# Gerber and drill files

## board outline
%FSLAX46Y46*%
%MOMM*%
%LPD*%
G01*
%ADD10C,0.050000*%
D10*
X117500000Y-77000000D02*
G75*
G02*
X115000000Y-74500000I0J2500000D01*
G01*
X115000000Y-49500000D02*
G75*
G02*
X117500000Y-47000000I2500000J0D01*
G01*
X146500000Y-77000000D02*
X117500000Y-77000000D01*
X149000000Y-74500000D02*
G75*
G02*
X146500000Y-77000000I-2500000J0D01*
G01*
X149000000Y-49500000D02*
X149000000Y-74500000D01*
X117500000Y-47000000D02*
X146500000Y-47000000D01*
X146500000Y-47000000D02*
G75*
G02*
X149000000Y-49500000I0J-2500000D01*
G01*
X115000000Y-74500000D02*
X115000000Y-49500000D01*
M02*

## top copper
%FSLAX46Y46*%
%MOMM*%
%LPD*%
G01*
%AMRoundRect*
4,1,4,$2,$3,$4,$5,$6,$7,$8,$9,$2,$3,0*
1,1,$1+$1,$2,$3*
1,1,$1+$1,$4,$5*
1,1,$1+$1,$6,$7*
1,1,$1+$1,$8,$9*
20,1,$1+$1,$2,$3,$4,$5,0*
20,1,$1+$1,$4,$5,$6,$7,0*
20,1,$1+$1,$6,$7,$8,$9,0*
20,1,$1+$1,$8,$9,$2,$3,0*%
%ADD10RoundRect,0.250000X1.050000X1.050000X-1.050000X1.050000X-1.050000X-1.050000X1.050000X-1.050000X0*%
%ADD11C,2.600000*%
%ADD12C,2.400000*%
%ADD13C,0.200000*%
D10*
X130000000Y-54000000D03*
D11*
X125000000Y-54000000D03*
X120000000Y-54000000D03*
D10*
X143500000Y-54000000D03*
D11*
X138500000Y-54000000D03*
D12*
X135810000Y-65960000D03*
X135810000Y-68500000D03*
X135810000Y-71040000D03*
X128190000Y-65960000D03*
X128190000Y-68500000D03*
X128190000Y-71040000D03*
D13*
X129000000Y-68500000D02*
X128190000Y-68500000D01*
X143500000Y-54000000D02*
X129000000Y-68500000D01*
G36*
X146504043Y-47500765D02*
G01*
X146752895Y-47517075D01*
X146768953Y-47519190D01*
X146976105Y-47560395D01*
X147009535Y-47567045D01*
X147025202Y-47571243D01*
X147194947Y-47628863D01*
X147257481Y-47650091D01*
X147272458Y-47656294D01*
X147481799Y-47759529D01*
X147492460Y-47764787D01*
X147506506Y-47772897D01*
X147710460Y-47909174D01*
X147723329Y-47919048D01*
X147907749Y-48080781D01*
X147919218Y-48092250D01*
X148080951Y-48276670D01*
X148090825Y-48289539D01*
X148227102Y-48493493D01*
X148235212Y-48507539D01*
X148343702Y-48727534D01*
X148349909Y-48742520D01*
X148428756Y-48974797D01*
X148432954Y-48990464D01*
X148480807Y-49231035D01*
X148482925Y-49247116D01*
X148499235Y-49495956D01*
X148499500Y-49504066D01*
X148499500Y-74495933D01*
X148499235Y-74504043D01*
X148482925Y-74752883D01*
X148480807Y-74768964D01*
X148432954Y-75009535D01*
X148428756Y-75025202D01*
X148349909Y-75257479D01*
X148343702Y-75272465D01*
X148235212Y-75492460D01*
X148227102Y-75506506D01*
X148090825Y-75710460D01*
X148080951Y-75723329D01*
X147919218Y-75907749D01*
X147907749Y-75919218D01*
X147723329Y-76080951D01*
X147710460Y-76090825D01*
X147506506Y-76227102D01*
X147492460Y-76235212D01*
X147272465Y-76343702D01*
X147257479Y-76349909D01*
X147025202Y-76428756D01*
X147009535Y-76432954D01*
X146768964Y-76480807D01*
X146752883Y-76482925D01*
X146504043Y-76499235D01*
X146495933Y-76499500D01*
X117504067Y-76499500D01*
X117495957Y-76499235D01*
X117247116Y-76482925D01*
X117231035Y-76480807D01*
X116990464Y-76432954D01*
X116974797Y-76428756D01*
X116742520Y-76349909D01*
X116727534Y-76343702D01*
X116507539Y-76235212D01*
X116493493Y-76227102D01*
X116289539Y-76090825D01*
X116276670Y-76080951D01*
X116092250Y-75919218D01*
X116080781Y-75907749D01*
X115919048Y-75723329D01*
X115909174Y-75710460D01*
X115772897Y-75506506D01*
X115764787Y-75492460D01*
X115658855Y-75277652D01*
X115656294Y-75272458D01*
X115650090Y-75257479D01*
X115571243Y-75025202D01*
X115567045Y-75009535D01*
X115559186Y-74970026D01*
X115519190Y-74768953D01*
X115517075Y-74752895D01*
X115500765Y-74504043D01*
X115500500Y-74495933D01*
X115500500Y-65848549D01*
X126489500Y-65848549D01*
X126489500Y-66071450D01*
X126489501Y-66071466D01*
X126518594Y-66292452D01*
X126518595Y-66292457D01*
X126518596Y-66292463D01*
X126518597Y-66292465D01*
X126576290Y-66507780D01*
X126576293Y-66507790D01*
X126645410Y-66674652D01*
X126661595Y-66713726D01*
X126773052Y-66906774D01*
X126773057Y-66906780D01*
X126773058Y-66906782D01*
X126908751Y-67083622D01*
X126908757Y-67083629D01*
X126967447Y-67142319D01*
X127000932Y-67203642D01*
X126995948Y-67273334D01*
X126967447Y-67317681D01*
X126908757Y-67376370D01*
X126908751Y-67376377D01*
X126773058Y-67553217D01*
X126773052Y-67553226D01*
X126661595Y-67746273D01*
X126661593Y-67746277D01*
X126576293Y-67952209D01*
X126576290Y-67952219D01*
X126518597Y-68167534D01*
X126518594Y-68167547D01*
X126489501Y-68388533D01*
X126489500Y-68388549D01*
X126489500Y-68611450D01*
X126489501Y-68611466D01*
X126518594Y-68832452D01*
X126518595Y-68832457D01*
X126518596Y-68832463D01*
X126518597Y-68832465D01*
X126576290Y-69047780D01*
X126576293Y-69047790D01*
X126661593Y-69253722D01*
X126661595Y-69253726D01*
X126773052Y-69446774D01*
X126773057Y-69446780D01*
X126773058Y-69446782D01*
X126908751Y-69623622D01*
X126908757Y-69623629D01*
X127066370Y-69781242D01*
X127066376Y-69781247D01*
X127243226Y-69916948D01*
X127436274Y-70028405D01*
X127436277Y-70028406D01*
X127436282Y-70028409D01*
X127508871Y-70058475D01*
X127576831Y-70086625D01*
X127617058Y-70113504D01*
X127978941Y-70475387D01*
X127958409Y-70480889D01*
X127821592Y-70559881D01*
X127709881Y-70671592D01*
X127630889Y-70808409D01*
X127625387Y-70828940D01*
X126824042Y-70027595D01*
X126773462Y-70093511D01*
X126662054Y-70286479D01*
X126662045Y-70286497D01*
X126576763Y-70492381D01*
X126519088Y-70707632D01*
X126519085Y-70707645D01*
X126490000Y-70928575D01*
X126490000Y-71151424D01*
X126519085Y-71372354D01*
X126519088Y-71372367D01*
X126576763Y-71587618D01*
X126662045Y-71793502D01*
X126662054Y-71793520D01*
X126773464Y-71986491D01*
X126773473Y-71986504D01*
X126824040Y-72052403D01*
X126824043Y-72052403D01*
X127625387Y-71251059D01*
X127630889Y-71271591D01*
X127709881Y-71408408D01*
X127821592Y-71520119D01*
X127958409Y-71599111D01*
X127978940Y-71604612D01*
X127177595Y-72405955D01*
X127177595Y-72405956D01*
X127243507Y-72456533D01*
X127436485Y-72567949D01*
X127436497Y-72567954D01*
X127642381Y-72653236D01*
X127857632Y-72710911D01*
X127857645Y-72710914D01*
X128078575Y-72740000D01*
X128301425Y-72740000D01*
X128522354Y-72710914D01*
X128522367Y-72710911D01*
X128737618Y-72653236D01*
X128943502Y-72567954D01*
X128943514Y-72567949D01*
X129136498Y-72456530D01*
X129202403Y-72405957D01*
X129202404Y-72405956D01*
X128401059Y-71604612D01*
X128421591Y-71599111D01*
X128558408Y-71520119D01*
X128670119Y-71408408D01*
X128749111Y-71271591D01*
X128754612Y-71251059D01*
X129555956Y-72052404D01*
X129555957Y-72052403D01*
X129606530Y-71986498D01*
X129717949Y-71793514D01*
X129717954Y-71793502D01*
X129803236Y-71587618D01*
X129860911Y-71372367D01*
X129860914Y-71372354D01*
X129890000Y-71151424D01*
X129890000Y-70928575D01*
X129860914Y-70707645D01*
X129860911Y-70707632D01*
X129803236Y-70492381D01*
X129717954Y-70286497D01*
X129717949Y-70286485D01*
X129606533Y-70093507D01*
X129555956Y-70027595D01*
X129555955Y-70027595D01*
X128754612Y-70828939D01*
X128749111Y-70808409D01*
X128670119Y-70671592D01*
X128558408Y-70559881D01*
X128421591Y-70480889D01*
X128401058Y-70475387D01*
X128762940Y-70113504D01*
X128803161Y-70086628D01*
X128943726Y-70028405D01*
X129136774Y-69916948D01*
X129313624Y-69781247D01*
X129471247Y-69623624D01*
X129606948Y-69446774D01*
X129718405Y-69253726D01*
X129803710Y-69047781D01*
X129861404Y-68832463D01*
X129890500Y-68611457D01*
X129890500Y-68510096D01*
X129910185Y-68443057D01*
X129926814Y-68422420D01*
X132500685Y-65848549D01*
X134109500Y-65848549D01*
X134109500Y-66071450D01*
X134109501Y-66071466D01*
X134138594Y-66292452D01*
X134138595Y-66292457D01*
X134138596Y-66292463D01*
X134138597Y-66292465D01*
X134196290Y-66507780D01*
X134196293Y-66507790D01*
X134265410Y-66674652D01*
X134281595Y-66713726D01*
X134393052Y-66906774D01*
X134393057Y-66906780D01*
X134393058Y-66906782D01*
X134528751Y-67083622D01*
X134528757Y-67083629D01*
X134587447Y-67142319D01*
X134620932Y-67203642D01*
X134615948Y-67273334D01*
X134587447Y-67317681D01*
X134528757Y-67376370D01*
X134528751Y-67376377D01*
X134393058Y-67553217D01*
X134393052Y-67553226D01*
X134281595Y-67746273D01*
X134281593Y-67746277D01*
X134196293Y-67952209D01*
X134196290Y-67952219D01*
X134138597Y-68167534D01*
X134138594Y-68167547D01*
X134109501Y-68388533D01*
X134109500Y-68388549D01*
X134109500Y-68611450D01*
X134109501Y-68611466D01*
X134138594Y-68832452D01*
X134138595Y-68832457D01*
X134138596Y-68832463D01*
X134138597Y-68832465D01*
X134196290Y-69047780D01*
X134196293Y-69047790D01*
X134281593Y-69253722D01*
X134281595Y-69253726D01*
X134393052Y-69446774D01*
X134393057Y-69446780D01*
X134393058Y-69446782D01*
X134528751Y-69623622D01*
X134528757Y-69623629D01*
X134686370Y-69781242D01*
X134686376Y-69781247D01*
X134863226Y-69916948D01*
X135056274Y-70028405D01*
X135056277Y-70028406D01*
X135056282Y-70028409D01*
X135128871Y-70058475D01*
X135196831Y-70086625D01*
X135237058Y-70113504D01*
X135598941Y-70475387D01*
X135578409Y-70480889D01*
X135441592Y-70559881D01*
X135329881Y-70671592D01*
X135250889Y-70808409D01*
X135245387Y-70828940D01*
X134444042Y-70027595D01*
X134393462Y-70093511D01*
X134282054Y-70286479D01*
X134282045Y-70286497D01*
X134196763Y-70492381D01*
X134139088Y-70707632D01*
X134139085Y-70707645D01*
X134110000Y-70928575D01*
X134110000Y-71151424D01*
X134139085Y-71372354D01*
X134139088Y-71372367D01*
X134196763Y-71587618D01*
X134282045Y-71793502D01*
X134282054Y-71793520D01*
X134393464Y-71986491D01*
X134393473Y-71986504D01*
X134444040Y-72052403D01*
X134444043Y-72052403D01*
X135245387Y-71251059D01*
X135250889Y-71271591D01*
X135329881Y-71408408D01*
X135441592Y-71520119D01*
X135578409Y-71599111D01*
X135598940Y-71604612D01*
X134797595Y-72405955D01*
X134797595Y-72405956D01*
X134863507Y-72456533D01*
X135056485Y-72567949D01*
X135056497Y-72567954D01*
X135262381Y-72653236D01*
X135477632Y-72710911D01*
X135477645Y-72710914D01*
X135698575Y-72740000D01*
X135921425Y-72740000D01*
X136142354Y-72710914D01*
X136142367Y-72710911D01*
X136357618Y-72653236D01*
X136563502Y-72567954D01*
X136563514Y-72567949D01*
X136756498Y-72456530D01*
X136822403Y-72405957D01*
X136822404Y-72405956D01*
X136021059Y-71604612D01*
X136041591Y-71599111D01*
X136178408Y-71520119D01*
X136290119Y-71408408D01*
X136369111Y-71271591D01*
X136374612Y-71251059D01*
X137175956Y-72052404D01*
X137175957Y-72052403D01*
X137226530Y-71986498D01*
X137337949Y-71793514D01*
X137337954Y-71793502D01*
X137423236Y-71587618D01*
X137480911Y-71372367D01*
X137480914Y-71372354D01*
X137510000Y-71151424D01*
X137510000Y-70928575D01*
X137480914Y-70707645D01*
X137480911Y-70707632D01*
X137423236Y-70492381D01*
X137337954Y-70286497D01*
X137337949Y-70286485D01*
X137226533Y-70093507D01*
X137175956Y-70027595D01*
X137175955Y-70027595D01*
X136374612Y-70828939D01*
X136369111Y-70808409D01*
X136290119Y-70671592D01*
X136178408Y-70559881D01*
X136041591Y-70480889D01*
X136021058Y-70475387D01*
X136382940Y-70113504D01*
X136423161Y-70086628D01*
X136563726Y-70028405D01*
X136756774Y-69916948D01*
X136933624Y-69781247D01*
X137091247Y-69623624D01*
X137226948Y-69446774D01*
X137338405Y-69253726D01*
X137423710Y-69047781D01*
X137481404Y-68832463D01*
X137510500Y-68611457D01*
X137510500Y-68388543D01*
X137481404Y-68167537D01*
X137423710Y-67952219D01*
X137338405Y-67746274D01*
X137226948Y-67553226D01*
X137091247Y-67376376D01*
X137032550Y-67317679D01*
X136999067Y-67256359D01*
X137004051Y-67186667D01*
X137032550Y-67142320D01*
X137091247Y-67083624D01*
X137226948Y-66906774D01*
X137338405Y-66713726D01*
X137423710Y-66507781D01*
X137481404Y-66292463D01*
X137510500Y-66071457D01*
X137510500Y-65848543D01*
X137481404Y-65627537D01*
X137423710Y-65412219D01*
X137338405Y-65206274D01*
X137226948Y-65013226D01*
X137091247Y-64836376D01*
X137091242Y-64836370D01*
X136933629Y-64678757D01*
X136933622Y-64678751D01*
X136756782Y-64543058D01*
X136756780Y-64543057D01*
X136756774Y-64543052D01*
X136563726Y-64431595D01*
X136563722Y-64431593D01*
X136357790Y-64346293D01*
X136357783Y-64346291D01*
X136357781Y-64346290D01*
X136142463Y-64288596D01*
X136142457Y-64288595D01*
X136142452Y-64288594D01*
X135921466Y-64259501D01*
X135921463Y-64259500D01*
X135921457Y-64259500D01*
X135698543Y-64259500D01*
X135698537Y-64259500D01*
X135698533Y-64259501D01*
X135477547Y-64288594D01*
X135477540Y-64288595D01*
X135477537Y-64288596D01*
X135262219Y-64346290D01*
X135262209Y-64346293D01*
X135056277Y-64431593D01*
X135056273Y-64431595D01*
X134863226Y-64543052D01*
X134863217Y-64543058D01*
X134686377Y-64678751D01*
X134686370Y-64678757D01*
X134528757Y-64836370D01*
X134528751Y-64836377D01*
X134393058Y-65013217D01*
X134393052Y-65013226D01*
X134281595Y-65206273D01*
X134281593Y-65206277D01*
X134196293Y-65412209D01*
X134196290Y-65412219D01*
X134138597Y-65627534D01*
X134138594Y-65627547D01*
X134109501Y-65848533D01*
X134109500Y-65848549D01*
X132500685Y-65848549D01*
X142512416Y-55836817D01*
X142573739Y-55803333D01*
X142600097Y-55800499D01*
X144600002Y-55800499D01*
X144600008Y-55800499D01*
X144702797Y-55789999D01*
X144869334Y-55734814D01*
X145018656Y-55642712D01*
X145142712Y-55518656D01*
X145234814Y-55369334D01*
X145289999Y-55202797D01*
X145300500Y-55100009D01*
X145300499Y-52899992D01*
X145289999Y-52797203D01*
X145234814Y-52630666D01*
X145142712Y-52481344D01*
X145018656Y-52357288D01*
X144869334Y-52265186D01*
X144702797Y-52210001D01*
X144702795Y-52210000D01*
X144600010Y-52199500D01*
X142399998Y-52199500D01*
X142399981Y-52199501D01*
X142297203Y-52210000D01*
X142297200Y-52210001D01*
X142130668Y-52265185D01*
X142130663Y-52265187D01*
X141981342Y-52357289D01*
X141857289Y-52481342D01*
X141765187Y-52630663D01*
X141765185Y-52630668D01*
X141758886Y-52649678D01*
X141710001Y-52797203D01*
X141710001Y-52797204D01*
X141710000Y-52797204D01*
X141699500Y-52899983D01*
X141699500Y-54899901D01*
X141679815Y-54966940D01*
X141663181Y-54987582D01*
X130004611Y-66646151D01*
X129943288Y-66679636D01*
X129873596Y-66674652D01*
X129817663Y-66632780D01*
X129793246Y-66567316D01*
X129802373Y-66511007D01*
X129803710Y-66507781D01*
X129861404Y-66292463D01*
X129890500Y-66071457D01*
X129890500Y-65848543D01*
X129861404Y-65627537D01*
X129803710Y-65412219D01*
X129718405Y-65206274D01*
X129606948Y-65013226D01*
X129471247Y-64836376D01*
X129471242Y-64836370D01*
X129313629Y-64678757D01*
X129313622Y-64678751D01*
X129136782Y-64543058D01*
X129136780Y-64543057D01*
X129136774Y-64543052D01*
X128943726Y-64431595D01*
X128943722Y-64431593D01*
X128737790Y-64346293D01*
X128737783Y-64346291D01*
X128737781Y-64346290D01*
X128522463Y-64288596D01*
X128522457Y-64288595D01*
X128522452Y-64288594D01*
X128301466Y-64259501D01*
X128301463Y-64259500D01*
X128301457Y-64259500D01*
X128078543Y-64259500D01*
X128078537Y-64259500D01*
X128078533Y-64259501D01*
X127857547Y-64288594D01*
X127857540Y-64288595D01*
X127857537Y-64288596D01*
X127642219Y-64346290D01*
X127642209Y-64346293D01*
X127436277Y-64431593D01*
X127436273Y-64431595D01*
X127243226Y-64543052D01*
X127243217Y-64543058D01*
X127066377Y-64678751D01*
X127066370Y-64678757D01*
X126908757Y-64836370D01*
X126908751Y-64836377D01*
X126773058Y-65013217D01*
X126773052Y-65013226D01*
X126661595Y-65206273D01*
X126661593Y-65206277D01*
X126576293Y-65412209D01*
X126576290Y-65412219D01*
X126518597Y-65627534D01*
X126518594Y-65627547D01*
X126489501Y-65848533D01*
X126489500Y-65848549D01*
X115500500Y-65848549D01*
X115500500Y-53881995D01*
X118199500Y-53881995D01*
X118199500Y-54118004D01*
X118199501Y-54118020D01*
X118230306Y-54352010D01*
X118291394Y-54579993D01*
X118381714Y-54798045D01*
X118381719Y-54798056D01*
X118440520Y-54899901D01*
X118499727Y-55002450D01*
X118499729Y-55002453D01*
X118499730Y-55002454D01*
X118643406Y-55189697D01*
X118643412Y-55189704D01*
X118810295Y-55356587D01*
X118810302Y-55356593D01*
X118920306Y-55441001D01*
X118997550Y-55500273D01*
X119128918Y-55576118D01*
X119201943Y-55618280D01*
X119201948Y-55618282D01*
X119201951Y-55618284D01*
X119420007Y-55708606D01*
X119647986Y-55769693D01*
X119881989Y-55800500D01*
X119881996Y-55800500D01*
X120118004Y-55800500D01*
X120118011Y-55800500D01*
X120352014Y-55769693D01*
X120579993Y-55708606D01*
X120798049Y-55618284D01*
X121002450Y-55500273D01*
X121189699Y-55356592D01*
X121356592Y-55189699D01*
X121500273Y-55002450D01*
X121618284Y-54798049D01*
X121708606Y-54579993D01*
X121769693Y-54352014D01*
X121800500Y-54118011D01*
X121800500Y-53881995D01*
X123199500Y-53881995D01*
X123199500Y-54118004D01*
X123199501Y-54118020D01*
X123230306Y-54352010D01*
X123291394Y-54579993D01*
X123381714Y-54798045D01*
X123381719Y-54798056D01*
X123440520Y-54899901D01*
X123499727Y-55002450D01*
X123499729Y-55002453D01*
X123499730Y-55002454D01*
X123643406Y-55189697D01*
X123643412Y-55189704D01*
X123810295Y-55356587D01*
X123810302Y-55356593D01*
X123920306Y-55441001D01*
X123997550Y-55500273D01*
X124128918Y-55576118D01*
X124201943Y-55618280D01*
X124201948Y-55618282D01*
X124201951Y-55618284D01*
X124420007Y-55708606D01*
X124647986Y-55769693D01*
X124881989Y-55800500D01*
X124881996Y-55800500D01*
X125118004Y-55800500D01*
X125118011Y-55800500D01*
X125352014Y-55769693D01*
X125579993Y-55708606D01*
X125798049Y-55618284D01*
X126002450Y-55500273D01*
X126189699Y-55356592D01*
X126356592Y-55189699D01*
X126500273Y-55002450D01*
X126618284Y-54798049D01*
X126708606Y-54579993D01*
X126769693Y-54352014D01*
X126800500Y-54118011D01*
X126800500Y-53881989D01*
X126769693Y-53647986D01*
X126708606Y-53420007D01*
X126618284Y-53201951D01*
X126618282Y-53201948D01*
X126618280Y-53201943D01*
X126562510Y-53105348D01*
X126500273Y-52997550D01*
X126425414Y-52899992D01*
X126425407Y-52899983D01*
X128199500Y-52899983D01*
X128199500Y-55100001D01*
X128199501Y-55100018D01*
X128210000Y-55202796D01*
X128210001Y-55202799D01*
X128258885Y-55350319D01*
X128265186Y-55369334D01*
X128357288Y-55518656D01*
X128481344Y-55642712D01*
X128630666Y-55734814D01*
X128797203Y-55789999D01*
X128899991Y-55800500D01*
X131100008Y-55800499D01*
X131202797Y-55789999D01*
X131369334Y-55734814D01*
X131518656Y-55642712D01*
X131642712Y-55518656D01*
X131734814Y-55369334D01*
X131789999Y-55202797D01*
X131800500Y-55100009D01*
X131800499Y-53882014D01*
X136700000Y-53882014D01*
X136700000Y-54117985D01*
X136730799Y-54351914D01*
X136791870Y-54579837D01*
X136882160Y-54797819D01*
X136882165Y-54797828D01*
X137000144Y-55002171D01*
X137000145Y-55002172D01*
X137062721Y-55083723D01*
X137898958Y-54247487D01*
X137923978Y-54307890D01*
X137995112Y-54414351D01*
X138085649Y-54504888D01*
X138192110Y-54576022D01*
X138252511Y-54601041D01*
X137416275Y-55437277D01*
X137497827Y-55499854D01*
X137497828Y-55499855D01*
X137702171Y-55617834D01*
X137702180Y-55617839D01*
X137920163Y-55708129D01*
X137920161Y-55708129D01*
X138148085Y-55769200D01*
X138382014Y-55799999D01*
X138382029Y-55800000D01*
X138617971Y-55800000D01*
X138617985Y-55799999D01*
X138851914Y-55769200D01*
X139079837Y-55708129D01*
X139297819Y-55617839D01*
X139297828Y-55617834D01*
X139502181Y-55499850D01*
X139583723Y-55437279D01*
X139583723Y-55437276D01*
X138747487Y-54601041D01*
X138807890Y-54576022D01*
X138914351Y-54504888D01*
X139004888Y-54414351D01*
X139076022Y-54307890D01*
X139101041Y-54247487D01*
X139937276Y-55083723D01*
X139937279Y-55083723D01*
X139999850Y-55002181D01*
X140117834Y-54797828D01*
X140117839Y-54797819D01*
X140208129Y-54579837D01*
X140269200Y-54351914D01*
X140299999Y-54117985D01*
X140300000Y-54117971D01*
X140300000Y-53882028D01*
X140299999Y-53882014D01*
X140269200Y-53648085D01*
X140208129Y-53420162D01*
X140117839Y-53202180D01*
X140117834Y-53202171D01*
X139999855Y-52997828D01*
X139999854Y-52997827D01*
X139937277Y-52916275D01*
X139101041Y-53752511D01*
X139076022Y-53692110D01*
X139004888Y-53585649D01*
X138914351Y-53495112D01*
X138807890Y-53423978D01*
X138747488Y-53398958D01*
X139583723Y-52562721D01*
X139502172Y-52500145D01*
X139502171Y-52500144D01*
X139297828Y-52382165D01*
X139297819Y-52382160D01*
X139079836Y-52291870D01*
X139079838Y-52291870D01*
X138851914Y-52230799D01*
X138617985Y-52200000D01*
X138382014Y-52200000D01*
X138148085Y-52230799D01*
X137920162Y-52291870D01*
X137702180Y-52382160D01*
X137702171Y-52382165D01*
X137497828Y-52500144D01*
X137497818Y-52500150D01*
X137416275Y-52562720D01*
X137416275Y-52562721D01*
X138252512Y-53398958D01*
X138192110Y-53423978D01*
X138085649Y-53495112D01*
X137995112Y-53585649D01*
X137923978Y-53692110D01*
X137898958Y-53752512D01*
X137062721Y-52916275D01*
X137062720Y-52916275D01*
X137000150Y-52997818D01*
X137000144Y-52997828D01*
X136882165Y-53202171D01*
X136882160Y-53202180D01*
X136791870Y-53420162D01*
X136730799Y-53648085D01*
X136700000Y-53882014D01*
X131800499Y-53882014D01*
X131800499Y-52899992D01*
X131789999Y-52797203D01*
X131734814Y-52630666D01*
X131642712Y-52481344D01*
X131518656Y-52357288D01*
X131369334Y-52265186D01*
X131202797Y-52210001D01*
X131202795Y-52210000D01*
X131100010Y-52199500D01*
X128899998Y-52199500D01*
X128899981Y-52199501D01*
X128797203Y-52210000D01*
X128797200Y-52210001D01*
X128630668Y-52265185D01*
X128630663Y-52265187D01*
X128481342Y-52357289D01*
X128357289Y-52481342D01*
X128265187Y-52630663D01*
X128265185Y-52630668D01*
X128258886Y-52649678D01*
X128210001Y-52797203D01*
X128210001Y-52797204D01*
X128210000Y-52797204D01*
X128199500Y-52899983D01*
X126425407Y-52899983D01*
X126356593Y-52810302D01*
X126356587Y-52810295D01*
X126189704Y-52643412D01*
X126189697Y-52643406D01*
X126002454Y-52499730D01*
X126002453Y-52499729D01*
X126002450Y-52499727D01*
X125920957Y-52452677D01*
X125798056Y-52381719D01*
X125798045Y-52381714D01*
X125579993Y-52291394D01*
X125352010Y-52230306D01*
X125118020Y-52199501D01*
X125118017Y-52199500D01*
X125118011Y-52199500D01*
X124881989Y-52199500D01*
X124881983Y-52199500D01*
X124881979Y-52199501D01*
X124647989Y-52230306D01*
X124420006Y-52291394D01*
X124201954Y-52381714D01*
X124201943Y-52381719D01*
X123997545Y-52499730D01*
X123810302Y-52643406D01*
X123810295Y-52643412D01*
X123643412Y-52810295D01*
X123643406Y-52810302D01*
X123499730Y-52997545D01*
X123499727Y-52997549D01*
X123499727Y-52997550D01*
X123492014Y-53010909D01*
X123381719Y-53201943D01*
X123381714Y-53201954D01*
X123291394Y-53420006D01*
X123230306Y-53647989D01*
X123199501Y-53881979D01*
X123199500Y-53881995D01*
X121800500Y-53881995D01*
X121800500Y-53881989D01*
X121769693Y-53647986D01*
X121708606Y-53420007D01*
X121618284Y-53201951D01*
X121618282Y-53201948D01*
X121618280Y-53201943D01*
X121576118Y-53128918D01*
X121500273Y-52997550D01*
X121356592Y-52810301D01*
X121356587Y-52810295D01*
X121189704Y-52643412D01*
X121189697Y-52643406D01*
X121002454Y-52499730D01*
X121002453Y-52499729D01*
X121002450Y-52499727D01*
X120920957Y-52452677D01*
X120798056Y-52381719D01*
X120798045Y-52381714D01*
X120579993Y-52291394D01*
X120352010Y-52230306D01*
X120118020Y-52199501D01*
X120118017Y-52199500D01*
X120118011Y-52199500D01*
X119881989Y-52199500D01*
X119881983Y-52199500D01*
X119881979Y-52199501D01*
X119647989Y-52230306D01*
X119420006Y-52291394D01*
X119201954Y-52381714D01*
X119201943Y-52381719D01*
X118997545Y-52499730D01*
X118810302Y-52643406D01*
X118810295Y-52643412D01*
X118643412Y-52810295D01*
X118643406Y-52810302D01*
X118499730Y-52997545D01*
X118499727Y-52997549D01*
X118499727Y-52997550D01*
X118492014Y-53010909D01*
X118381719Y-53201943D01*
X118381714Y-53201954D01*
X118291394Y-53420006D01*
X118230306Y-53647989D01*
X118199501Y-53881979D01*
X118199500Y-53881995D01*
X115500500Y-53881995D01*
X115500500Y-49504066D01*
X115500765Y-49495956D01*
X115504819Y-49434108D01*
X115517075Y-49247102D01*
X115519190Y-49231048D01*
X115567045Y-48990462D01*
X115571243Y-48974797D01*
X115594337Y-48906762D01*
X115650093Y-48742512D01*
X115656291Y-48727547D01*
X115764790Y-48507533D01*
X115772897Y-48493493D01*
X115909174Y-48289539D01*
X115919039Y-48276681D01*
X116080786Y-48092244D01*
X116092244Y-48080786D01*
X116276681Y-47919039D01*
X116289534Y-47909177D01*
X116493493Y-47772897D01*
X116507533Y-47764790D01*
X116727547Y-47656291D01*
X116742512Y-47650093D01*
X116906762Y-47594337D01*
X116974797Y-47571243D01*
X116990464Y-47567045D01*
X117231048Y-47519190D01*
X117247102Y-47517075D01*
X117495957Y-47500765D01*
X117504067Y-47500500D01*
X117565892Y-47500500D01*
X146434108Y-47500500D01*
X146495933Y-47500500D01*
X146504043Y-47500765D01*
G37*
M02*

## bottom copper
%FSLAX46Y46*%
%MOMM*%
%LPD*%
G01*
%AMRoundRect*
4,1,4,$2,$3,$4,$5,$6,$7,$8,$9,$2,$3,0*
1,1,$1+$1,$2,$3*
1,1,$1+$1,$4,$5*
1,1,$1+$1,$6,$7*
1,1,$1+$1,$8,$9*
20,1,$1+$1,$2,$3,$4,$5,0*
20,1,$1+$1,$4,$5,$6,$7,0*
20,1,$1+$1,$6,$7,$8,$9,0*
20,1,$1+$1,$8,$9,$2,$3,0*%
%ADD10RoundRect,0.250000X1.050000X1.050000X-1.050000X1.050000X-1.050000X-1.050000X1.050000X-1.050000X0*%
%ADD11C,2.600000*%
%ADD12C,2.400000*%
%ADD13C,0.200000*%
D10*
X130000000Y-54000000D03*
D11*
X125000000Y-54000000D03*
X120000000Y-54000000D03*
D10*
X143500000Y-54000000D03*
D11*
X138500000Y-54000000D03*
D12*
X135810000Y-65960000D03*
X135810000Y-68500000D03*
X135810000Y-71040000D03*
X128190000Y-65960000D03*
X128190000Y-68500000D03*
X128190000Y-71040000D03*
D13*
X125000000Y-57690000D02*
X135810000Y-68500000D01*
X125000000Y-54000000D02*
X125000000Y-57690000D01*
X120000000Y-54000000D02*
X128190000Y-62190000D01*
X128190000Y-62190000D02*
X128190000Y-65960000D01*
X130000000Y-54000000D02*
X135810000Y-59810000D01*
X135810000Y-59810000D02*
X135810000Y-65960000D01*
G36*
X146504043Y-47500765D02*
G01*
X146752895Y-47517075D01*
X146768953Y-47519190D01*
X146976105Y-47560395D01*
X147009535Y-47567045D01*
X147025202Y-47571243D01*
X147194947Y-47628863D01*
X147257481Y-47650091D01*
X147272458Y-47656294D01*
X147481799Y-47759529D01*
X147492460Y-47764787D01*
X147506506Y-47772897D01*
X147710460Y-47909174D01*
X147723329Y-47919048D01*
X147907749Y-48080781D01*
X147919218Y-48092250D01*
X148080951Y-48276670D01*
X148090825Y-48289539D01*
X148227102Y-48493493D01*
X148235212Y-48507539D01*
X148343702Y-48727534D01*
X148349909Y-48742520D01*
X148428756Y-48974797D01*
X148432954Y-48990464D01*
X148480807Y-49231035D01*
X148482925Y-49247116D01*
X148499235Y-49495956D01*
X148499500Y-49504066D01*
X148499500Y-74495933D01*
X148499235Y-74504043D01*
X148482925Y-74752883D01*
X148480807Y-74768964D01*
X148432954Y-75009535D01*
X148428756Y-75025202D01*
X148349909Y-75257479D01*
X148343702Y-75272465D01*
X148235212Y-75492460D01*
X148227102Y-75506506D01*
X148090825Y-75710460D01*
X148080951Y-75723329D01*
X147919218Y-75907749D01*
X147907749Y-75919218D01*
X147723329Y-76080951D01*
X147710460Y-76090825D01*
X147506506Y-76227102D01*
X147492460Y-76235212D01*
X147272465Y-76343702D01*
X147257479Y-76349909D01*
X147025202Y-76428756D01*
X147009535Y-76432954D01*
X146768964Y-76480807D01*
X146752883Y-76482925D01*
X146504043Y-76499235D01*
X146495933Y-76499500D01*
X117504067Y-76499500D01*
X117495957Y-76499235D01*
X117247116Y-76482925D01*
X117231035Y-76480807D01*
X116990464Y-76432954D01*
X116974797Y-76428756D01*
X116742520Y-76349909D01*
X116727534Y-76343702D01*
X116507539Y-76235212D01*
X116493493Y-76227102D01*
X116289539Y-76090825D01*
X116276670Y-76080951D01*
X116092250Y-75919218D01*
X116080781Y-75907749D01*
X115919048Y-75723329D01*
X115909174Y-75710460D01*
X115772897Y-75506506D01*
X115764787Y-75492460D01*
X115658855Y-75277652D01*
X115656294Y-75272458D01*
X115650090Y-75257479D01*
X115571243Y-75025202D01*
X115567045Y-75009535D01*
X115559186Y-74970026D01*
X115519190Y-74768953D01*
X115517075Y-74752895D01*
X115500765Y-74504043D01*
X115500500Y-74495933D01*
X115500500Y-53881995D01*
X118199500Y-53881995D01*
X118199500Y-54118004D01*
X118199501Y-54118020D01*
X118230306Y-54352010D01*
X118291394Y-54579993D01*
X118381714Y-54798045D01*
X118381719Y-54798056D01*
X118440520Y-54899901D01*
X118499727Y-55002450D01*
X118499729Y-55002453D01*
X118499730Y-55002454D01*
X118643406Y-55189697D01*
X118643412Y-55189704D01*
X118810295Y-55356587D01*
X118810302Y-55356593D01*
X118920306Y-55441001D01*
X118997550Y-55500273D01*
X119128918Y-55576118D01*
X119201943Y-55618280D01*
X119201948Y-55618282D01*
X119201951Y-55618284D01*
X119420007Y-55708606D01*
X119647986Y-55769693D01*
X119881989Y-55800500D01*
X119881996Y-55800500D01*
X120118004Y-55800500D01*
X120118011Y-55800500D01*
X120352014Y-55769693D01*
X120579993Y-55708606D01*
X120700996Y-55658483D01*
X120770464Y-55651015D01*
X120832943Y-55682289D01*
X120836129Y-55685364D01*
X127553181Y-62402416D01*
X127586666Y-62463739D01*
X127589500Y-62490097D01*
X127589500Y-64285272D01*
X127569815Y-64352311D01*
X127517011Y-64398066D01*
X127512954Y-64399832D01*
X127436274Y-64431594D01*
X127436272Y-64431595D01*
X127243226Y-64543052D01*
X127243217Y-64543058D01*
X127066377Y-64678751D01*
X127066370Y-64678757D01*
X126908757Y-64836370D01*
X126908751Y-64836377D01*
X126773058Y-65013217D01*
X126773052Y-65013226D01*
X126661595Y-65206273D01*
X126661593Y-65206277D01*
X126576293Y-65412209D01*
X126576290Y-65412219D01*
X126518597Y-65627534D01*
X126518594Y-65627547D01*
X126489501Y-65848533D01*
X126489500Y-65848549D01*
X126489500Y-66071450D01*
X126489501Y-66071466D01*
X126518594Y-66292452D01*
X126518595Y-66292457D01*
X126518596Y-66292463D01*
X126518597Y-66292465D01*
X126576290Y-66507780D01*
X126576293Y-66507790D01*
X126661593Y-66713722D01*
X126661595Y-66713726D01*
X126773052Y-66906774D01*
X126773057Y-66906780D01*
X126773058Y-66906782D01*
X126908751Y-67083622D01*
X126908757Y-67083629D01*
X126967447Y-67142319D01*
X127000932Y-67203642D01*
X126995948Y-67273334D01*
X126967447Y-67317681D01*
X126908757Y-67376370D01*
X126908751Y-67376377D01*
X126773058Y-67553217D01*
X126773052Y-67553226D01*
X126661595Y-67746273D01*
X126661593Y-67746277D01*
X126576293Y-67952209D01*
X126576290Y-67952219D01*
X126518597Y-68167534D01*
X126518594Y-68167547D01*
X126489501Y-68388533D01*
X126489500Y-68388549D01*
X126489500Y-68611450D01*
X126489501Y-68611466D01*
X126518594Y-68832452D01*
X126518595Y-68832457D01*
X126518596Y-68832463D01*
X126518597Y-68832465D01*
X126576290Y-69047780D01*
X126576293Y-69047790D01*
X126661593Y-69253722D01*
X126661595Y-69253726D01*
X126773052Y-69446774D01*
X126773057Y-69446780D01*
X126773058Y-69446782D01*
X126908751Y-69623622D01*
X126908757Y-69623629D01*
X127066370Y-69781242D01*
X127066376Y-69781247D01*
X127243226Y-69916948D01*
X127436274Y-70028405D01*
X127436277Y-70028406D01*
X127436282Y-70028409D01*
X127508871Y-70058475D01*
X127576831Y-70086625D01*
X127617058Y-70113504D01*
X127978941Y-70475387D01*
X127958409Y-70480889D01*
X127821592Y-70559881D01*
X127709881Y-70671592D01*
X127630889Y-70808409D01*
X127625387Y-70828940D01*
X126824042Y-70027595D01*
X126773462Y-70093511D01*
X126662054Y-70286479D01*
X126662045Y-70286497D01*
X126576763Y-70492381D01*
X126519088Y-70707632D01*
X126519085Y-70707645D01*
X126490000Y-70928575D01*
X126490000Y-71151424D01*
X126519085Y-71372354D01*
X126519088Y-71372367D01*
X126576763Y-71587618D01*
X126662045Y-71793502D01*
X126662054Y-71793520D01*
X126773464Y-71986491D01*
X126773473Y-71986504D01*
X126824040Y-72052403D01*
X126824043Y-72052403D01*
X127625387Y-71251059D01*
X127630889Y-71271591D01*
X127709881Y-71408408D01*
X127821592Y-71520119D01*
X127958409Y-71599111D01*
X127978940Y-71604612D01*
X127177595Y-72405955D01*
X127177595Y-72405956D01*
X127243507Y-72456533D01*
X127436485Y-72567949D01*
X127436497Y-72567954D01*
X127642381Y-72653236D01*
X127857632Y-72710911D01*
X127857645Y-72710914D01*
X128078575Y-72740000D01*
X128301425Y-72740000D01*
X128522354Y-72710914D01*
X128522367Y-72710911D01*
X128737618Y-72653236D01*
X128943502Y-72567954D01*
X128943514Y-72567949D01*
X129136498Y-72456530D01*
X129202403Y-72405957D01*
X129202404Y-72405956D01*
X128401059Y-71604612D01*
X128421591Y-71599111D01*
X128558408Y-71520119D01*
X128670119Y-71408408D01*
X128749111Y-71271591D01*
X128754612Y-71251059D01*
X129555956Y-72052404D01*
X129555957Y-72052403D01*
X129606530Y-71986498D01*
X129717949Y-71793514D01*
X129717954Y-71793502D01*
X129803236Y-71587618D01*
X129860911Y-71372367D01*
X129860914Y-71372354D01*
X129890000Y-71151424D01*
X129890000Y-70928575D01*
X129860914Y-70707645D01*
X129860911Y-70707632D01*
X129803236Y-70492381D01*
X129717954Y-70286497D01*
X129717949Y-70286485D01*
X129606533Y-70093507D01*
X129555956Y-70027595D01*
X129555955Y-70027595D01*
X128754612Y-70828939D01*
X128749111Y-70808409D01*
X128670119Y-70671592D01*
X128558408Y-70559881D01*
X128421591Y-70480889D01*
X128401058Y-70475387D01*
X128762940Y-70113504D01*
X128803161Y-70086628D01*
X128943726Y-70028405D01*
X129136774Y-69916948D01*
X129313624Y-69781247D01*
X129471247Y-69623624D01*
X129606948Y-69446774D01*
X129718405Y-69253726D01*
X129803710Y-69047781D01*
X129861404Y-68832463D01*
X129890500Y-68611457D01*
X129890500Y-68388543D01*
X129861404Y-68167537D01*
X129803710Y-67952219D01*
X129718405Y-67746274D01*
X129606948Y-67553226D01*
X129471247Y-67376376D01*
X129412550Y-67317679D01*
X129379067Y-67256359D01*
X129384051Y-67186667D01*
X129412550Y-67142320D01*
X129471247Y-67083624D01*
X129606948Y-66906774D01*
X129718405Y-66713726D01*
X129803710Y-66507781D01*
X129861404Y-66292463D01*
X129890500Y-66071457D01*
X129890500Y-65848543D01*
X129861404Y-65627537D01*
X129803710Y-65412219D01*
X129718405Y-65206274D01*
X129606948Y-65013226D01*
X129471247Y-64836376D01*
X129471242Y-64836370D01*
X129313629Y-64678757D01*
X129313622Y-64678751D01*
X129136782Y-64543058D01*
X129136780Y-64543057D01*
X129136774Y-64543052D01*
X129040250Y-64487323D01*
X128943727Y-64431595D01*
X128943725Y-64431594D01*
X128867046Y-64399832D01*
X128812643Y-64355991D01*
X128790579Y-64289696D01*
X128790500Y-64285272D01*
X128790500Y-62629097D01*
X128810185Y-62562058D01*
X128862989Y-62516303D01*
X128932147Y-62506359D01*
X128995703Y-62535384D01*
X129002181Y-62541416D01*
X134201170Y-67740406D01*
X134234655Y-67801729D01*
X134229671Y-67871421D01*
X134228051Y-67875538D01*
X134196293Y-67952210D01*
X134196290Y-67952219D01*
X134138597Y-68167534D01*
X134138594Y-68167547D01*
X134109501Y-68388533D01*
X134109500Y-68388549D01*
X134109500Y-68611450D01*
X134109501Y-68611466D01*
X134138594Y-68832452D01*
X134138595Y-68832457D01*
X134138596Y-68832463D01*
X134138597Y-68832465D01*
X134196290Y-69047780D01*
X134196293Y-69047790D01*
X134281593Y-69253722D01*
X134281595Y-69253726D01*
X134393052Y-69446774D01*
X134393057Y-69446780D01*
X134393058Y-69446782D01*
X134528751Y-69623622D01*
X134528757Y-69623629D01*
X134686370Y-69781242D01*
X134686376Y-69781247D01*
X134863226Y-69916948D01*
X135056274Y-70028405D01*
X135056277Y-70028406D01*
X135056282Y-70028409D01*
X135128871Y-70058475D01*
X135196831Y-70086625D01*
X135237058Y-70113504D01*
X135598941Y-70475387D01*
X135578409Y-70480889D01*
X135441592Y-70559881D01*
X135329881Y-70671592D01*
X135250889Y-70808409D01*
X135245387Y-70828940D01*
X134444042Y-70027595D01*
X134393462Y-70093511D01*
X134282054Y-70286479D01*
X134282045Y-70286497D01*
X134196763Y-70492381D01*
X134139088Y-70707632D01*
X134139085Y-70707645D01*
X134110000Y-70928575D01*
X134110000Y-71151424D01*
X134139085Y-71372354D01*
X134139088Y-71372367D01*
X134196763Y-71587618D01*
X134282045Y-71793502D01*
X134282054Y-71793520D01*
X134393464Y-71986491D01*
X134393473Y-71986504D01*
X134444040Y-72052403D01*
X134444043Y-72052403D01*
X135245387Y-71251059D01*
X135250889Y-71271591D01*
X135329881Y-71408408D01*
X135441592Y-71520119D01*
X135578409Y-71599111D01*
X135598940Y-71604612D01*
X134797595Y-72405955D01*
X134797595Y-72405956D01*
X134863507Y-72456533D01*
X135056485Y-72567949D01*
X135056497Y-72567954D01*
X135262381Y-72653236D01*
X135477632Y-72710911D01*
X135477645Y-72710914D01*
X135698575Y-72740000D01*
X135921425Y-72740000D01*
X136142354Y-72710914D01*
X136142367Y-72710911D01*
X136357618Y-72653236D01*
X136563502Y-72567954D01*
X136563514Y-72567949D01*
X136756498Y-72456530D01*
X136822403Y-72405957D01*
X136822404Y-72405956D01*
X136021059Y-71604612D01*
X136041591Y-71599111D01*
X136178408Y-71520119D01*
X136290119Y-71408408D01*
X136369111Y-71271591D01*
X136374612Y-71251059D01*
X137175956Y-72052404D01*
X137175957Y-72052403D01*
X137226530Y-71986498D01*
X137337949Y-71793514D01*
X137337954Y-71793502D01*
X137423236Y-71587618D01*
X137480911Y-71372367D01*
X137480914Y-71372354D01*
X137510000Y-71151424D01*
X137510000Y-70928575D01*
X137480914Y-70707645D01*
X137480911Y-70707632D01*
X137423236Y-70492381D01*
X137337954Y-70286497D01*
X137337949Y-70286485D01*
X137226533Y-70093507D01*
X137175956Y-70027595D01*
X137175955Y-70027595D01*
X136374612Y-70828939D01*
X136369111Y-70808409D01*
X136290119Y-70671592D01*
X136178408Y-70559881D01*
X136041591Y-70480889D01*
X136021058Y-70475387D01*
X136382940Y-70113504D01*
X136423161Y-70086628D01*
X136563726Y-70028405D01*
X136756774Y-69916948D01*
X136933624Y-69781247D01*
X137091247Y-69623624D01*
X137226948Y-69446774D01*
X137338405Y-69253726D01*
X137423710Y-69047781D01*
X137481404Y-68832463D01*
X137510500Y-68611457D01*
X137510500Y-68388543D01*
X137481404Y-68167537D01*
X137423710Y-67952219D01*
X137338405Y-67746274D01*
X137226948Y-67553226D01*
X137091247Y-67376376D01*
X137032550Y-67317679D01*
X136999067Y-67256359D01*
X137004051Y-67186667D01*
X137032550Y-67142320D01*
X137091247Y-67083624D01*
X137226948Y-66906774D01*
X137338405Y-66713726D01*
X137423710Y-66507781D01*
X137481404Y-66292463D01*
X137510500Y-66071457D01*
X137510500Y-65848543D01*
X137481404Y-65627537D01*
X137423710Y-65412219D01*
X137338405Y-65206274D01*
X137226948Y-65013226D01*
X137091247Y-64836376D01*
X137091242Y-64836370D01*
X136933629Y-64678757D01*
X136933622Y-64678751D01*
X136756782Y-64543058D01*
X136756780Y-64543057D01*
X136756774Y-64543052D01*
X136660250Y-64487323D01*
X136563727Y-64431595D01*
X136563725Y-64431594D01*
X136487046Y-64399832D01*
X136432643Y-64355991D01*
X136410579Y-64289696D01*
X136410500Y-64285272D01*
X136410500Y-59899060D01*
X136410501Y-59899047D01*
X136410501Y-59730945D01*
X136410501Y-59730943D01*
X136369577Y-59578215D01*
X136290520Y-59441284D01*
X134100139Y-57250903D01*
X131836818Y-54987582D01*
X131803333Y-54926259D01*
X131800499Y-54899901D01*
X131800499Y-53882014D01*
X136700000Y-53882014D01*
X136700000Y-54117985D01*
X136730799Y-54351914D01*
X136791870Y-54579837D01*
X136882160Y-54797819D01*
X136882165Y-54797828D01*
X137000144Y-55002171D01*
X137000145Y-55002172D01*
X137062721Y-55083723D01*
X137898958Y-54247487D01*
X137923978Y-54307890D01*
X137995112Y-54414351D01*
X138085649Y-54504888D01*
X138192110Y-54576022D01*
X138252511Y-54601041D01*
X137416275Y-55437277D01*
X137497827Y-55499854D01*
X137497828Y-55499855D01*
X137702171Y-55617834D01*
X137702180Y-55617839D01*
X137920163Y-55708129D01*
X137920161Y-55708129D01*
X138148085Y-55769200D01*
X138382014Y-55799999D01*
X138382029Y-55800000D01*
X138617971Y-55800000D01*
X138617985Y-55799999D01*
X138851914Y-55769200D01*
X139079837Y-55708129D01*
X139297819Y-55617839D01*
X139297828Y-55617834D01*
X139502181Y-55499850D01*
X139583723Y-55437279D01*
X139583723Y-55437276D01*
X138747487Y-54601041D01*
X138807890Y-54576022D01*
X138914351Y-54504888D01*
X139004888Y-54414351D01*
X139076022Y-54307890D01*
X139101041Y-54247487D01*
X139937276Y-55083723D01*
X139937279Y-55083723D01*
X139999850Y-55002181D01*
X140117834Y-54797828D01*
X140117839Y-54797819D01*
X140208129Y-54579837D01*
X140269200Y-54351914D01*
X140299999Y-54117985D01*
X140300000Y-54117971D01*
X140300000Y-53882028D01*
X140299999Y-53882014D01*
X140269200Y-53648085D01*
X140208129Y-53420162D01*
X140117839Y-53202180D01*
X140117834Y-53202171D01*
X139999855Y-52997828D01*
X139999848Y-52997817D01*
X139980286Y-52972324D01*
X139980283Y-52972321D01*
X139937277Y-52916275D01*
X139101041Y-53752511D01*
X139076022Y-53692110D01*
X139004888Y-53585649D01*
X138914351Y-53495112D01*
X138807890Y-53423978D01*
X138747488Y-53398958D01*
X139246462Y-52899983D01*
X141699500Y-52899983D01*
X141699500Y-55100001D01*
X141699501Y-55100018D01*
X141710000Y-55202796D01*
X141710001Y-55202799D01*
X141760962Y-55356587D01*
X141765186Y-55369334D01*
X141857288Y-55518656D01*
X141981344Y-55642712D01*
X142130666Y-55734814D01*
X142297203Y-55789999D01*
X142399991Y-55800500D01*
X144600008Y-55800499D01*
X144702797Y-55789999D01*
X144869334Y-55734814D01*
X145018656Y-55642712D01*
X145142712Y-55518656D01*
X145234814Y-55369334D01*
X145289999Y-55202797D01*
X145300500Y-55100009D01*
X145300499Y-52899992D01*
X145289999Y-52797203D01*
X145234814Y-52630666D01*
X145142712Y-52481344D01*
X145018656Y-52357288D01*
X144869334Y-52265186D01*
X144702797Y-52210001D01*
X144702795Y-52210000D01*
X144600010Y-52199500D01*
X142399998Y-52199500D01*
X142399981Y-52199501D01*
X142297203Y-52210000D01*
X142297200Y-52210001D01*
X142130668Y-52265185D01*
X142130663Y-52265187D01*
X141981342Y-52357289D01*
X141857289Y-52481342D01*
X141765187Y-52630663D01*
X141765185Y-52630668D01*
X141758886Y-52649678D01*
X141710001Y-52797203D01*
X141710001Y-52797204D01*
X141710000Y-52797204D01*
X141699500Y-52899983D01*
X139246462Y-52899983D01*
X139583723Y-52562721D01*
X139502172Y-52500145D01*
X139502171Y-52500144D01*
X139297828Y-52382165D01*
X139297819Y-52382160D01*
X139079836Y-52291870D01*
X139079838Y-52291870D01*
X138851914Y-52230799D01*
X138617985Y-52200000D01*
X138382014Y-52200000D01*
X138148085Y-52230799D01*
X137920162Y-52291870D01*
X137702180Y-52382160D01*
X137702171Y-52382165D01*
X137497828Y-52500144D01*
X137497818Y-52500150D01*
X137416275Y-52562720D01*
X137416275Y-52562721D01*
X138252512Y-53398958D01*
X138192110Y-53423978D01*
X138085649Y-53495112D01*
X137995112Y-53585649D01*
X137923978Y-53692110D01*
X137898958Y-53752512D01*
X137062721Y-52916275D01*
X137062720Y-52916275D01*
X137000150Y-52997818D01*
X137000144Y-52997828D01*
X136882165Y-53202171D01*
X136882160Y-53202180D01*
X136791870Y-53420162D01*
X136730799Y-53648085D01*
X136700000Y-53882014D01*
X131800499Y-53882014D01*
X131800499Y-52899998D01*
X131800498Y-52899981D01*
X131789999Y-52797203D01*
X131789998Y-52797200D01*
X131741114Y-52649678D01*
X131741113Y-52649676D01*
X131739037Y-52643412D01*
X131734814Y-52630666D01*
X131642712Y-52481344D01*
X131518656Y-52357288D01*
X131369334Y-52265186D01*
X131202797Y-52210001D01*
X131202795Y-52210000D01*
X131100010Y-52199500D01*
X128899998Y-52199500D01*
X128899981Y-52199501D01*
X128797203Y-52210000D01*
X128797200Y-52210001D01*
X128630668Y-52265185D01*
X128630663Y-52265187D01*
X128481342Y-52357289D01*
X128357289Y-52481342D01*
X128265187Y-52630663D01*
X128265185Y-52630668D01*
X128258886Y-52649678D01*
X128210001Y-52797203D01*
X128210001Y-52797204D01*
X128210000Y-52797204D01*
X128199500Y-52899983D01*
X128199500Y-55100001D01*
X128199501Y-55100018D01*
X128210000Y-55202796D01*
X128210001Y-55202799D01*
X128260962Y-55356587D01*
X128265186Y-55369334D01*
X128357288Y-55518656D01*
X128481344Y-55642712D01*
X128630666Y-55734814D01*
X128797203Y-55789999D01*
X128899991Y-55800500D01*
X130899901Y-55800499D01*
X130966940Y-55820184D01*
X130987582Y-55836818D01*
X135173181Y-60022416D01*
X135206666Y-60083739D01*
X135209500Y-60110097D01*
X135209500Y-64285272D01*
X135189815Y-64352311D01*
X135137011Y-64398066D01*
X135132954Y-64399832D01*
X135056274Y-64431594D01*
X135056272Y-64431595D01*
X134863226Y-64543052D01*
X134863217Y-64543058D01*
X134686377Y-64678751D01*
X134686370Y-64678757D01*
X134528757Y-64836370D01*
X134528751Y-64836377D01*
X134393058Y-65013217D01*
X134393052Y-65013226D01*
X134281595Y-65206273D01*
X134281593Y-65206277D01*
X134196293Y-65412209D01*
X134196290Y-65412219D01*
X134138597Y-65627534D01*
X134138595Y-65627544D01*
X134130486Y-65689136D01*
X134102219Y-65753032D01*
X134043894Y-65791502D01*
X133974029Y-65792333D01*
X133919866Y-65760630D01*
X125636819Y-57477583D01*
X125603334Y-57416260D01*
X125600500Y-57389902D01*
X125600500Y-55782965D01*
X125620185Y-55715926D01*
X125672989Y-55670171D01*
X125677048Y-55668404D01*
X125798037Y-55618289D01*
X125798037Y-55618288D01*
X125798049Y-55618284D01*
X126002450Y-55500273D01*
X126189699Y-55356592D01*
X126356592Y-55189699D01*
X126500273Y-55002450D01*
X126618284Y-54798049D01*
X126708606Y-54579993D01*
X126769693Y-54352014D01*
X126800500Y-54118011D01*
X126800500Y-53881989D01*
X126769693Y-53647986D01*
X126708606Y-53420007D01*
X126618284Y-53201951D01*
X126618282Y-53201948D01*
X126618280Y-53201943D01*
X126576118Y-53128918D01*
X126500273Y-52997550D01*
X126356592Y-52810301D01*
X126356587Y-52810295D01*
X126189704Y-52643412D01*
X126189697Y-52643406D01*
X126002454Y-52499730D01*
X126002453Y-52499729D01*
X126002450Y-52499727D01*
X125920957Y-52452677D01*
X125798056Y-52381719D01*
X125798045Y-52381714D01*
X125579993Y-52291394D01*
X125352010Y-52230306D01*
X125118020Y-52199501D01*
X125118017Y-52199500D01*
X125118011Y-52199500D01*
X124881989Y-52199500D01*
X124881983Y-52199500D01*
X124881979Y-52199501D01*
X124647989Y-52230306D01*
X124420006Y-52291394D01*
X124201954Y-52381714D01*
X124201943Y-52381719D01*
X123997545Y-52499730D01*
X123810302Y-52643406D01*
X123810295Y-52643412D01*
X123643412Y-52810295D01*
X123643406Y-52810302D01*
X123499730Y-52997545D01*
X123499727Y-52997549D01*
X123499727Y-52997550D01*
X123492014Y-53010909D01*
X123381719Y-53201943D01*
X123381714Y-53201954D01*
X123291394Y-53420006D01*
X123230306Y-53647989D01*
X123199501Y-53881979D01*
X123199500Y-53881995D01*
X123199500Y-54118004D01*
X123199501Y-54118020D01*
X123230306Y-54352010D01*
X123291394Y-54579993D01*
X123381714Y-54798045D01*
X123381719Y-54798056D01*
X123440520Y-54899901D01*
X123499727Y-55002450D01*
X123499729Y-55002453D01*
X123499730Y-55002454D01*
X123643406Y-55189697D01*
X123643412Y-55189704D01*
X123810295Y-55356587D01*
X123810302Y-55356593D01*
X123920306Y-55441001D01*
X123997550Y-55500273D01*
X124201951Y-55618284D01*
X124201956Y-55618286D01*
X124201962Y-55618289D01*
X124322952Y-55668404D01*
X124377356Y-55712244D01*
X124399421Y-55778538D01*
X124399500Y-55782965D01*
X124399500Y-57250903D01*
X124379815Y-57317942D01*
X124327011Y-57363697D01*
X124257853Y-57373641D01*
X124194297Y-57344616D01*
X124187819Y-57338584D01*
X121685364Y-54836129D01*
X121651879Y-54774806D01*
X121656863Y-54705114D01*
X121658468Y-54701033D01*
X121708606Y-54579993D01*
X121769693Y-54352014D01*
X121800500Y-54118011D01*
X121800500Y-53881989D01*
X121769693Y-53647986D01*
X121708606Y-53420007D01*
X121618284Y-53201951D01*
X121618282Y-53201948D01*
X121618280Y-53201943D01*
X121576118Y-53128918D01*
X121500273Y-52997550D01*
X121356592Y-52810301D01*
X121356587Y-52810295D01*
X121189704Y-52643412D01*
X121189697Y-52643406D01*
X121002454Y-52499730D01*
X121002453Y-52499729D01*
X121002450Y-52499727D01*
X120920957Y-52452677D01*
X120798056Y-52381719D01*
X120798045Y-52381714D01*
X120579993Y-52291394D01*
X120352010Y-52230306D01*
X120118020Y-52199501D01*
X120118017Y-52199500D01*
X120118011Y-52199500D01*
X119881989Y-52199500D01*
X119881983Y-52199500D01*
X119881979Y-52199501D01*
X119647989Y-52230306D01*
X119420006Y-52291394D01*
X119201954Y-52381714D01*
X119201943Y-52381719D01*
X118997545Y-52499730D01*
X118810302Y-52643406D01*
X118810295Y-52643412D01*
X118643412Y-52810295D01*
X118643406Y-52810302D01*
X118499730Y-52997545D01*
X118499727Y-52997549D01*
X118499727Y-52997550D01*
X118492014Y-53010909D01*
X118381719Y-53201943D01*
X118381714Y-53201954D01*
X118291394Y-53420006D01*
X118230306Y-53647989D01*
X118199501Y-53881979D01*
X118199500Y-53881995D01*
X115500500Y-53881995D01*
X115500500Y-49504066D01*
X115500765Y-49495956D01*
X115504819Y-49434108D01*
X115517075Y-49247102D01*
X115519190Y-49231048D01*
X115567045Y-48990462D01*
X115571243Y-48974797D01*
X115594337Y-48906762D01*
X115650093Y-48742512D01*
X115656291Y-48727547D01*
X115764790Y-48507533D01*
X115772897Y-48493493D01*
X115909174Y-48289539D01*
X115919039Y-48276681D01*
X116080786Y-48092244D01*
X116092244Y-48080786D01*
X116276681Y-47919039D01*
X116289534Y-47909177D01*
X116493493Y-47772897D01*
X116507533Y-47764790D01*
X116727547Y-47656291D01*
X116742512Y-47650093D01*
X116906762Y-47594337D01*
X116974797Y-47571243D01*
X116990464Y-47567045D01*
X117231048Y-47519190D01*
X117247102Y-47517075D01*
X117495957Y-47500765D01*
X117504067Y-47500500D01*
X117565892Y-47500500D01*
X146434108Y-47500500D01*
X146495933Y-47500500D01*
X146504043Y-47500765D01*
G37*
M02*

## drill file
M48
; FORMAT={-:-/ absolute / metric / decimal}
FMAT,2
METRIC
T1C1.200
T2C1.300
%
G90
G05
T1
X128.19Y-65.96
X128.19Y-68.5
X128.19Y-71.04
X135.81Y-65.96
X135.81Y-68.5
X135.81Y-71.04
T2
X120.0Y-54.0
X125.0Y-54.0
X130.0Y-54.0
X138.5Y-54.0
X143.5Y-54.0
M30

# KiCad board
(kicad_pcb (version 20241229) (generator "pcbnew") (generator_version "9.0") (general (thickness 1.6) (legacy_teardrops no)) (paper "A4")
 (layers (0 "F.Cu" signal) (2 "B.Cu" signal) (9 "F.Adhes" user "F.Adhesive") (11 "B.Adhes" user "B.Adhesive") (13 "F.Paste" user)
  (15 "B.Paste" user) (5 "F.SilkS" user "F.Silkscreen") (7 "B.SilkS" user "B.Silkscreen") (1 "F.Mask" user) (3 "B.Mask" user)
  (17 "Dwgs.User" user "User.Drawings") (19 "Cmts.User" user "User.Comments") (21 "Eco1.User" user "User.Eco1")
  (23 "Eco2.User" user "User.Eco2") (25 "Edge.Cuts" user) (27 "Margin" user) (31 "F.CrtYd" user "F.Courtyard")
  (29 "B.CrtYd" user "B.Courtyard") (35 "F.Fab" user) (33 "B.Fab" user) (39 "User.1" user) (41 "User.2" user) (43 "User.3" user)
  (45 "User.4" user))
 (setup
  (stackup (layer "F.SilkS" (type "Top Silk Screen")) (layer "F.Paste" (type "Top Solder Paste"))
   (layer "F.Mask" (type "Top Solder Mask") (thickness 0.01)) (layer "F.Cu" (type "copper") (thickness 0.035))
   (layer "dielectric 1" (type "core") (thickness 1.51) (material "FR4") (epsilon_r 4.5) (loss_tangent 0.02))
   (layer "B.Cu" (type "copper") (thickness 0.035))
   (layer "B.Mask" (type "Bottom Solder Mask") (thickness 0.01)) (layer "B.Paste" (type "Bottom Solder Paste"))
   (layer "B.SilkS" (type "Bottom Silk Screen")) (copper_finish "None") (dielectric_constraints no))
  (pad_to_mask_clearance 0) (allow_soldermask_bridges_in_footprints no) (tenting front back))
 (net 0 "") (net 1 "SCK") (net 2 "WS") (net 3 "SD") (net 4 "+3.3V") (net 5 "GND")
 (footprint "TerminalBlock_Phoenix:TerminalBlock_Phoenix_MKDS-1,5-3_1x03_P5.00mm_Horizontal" (layer "F.Cu") (at 130 54 180)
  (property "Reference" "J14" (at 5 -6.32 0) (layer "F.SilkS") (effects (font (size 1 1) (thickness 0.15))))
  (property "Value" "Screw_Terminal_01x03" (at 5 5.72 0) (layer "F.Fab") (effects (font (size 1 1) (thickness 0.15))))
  (pad "1" thru_hole roundrect (at 0 0 180) (size 2.6 2.6) (drill 1.3) (layers "*.Cu" "*.Mask") (remove_unused_layers no)
   (roundrect_rratio 0.096154) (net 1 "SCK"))
  (pad "2" thru_hole circle (at 5 0 180) (size 2.6 2.6) (drill 1.3) (layers "*.Cu" "*.Mask") (remove_unused_layers no) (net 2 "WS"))
  (pad "3" thru_hole circle (at 10 0 180) (size 2.6 2.6) (drill 1.3) (layers "*.Cu" "*.Mask") (remove_unused_layers no) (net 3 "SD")))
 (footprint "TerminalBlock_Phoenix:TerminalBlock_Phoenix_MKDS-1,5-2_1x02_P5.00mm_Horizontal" (layer "F.Cu") (at 143.5 54 180)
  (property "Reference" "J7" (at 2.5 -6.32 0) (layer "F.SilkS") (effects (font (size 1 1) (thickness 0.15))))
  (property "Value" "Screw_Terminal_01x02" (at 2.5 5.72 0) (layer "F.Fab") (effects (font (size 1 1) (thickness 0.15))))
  (pad "1" thru_hole roundrect (at 0 0 180) (size 2.6 2.6) (drill 1.3) (layers "*.Cu" "*.Mask") (remove_unused_layers no)
   (roundrect_rratio 0.096154) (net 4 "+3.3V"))
  (pad "2" thru_hole circle (at 5 0 180) (size 2.6 2.6) (drill 1.3) (layers "*.Cu" "*.Mask") (remove_unused_layers no) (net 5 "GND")))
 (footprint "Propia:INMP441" (layer "F.Cu") (at 132 68.5)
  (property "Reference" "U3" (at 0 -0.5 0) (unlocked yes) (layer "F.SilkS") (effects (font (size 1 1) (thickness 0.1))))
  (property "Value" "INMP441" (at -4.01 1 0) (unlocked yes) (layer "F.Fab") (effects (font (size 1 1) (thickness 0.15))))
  (pad "1" thru_hole circle (at 3.81 -2.54) (size 2.4 2.4) (drill 1.2) (layers "*.Cu" "*.Mask") (remove_unused_layers no) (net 1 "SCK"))
  (pad "2" thru_hole circle (at 3.81 0) (size 2.4 2.4) (drill 1.2) (layers "*.Cu" "*.Mask") (remove_unused_layers no) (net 2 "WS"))
  (pad "3" thru_hole circle (at 3.81 2.54) (size 2.4 2.4) (drill 1.2) (layers "*.Cu" "*.Mask") (remove_unused_layers no) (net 5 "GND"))
  (pad "4" thru_hole circle (at -3.81 -2.54) (size 2.4 2.4) (drill 1.2) (layers "*.Cu" "*.Mask") (remove_unused_layers no) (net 3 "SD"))
  (pad "5" thru_hole circle (at -3.81 0) (size 2.4 2.4) (drill 1.2) (layers "*.Cu" "*.Mask") (remove_unused_layers no) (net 4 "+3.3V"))
  (pad "6" thru_hole circle (at -3.81 2.54) (size 2.4 2.4) (drill 1.2) (layers "*.Cu" "*.Mask") (remove_unused_layers no) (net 5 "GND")))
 (gr_arc (start 117.5 77) (mid 115.732233 76.267767) (end 115 74.5) (stroke (width 0.05) (type default)) (layer "Edge.Cuts"))
 (gr_arc (start 115 49.5) (mid 115.732233 47.732233) (end 117.5 47) (stroke (width 0.05) (type default)) (layer "Edge.Cuts"))
 (gr_line (start 146.5 77) (end 117.5 77) (stroke (width 0.05) (type default)) (layer "Edge.Cuts"))
 (gr_arc (start 149 74.5) (mid 148.267767 76.267767) (end 146.5 77) (stroke (width 0.05) (type default)) (layer "Edge.Cuts"))
 (gr_line (start 149 49.5) (end 149 74.5) (stroke (width 0.05) (type default)) (layer "Edge.Cuts"))
 (gr_line (start 117.5 47) (end 146.5 47) (stroke (width 0.05) (type default)) (layer "Edge.Cuts"))
 (gr_arc (start 146.5 47) (mid 148.267767 47.732233) (end 149 49.5) (stroke (width 0.05) (type default)) (layer "Edge.Cuts"))
 (gr_line (start 115 74.5) (end 115 49.5) (stroke (width 0.05) (type default)) (layer "Edge.Cuts"))
 (segment (start 129 68.5) (end 128.19 68.5) (width 0.2) (layer "F.Cu") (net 4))
 (segment (start 143.5 54) (end 129 68.5) (width 0.2) (layer "F.Cu") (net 4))
 (segment (start 125 57.69) (end 135.81 68.5) (width 0.2) (layer "B.Cu") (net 2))
 (segment (start 125 54) (end 125 57.69) (width 0.2) (layer "B.Cu") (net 2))
 (segment (start 120 54) (end 128.19 62.19) (width 0.2) (layer "B.Cu") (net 3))
 (segment (start 128.19 62.19) (end 128.19 65.96) (width 0.2) (layer "B.Cu") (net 3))
 (segment (start 130 54) (end 135.81 59.81) (width 0.2) (layer "B.Cu") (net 1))
 (segment (start 135.81 59.81) (end 135.81 65.96) (width 0.2) (layer "B.Cu") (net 1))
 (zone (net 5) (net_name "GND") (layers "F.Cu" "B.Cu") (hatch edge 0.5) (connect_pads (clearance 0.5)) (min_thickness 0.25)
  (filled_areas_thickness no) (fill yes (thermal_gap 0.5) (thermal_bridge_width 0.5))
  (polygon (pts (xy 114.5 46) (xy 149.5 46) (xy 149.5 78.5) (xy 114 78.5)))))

